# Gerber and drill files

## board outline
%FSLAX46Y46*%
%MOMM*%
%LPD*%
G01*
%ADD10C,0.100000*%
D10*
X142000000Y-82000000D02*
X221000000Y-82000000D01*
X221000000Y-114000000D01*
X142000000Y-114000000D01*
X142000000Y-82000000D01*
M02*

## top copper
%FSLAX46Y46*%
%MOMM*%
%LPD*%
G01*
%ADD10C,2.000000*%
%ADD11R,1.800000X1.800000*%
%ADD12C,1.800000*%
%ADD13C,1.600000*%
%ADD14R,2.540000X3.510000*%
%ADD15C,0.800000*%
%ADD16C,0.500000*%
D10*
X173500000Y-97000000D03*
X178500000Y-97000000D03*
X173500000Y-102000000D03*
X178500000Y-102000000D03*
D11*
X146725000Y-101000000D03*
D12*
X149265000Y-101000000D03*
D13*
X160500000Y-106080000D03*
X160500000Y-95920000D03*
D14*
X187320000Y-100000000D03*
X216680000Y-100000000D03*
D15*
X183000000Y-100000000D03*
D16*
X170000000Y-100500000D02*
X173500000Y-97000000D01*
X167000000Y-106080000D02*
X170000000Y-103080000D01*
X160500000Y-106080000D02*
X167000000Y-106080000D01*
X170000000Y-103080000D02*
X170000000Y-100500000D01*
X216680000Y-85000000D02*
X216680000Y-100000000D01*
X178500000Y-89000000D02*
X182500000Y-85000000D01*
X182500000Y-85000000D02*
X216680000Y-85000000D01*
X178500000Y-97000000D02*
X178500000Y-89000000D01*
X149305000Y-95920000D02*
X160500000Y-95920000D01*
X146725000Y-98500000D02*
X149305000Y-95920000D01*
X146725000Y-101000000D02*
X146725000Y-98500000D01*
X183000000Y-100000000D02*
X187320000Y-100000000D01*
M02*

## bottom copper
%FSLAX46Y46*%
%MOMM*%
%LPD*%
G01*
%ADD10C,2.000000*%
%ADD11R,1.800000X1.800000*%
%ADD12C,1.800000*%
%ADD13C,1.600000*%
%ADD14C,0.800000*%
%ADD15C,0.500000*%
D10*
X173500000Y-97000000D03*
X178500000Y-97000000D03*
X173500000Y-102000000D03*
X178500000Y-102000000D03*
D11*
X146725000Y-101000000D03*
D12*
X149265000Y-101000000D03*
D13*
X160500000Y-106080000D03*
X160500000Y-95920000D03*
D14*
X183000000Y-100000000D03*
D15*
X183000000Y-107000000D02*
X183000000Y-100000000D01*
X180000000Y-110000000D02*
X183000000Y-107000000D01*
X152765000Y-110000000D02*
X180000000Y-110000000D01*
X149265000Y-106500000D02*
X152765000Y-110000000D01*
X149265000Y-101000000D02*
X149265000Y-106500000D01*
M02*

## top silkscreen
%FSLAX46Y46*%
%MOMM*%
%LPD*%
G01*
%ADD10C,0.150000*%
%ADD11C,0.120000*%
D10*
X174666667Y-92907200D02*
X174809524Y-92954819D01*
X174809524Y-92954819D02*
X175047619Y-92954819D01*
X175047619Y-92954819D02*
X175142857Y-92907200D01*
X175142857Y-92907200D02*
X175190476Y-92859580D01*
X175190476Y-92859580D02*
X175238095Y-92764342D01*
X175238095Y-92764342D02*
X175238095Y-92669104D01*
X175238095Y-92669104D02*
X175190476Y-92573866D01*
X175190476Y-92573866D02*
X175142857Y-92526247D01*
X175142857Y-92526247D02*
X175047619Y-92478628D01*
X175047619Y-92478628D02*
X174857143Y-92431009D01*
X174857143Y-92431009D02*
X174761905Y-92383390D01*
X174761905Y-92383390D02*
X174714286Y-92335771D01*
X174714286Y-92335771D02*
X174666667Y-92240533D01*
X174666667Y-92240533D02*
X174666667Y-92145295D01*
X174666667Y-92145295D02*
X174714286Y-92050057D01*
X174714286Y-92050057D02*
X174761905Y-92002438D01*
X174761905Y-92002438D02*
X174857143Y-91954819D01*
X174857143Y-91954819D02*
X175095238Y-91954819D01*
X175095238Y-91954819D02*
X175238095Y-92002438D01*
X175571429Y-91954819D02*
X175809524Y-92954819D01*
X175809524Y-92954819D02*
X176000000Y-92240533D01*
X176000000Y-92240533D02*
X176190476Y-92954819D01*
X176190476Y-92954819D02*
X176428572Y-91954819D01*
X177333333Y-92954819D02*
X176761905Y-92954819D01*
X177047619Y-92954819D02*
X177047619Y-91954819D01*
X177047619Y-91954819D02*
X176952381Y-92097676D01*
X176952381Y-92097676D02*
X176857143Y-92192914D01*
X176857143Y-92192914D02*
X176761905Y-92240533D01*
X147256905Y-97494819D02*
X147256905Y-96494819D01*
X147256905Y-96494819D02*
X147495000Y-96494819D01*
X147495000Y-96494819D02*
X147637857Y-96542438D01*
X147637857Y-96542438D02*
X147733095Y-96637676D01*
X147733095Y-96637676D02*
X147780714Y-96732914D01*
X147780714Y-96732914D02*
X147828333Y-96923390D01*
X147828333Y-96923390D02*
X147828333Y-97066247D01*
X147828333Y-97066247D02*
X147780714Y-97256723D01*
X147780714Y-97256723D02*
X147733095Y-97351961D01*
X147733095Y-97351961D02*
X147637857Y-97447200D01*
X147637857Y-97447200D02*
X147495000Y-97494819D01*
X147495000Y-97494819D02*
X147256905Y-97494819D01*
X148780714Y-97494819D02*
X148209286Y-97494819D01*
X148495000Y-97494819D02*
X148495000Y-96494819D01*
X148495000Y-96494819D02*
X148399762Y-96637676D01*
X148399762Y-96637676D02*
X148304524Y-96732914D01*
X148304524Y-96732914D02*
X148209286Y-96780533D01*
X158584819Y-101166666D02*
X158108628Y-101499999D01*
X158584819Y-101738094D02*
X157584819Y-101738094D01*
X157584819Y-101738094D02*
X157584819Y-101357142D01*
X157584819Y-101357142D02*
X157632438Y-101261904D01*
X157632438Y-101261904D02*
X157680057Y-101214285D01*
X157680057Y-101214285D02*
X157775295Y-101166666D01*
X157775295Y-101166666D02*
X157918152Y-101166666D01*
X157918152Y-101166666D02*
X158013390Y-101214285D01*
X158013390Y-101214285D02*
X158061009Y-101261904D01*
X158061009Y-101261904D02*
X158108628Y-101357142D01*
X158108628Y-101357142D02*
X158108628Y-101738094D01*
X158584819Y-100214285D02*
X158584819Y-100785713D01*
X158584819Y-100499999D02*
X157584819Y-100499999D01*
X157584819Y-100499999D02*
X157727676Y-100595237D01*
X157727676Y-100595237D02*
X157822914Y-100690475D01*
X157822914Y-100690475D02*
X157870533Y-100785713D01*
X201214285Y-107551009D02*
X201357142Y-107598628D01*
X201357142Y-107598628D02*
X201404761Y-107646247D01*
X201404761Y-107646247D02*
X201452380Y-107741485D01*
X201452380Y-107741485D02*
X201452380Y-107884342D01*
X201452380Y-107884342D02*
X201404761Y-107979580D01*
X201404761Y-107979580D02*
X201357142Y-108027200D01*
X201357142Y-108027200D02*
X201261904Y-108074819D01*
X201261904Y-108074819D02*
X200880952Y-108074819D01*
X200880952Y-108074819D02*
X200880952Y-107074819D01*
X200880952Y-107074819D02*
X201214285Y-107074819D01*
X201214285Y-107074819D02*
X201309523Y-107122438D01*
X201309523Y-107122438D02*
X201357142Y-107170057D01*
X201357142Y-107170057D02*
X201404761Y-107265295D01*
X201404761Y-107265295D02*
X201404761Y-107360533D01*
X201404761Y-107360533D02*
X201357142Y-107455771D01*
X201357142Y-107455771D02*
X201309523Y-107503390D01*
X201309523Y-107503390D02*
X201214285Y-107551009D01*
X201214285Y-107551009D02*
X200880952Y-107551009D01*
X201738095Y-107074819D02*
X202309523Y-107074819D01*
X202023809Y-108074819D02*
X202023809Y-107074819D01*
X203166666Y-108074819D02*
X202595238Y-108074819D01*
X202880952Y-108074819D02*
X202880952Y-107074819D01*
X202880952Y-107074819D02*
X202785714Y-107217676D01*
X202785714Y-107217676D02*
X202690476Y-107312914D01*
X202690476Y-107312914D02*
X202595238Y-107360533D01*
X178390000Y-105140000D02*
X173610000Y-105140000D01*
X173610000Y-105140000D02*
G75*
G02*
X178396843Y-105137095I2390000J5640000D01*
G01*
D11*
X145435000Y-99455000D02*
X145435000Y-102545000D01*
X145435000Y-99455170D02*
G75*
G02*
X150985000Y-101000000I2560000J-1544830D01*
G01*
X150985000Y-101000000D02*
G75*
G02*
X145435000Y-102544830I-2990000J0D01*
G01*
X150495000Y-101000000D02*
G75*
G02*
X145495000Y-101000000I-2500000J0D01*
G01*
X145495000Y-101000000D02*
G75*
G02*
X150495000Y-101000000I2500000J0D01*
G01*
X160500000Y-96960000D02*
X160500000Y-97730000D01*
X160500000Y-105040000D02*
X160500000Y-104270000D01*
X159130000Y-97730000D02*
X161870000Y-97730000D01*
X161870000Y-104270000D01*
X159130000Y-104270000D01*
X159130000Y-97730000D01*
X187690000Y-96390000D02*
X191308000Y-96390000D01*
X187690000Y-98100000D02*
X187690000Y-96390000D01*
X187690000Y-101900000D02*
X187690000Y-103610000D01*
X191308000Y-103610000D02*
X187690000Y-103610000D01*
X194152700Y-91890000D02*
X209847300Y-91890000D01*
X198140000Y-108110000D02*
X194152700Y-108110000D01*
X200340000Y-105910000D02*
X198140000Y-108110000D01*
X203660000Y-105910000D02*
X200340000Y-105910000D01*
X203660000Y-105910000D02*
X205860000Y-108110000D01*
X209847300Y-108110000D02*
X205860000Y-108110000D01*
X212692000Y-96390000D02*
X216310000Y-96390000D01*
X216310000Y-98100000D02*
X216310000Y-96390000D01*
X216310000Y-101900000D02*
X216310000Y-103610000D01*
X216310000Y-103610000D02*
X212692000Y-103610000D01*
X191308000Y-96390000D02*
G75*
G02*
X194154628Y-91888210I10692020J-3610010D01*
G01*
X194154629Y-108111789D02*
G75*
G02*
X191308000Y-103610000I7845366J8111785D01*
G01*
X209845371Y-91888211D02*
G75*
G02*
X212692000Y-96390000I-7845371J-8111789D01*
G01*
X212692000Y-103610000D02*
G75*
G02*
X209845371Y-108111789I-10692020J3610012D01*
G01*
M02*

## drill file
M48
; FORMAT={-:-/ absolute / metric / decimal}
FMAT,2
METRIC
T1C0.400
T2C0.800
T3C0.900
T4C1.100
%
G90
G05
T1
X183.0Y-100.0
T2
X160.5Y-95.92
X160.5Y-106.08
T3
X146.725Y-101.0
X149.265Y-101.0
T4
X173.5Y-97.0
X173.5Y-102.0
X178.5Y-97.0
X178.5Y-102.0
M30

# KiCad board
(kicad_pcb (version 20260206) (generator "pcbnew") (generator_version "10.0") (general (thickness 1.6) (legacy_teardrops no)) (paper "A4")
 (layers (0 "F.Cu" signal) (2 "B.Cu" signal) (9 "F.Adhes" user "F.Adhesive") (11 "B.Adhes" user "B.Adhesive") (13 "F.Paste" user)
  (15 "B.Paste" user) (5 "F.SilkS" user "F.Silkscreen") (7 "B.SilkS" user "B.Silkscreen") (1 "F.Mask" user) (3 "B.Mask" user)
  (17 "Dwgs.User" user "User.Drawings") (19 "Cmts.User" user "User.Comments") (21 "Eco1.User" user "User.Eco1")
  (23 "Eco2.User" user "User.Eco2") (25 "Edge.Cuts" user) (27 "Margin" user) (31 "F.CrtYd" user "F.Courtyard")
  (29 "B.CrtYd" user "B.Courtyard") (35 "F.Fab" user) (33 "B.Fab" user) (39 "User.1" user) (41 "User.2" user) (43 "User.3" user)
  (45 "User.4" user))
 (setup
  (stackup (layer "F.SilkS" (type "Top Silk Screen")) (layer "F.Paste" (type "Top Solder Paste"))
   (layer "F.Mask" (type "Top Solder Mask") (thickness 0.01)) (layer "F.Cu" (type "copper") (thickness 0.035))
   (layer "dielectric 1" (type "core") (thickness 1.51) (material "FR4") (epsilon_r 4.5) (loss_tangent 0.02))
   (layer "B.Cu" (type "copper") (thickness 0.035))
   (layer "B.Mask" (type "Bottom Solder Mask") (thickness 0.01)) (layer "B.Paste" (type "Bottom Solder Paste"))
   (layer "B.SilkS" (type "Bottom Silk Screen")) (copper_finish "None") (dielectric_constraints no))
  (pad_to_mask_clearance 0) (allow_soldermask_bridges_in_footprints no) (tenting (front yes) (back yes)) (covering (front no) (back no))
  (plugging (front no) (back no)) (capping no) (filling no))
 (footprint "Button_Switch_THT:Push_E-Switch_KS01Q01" (layer "F.Cu") (at 173.5 97)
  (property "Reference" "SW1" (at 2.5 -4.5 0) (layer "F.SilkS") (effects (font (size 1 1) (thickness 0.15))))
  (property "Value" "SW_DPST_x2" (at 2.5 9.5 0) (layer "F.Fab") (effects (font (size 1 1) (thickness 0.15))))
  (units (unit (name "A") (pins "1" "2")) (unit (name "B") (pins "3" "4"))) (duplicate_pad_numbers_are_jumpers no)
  (fp_line (start 4.89 8.14) (end 0.11 8.14) (stroke (width 0.15) (type solid)) (layer "F.SilkS"))
  (fp_arc (start 0.11 8.14) (mid 2.496283 -3.625495) (end 4.896843 8.137095) (stroke (width 0.15) (type solid)) (layer "F.SilkS"))
  (pad "1" thru_hole circle (at 0 0) (size 2 2) (drill 1.1) (layers "*.Cu" "*.Mask") (remove_unused_layers no) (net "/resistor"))
  (pad "2" thru_hole circle (at 5 0) (size 2 2) (drill 1.1) (layers "*.Cu" "*.Mask") (remove_unused_layers no) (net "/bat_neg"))
  (pad "3" thru_hole circle (at 0 5) (size 2 2) (drill 1.1) (layers "*.Cu" "*.Mask") (remove_unused_layers no)
   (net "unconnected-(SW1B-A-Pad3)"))
  (pad "4" thru_hole circle (at 5 5) (size 2 2) (drill 1.1) (layers "*.Cu" "*.Mask") (remove_unused_layers no)
   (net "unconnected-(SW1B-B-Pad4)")))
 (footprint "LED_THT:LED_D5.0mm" (layer "F.Cu") (at 146.725 101)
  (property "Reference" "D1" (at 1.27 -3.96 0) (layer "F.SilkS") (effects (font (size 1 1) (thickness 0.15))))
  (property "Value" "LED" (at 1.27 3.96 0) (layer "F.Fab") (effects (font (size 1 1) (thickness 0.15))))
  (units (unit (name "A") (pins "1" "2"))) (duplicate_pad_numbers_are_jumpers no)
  (fp_line (start -1.29 -1.545) (end -1.29 1.545) (stroke (width 0.12) (type solid)) (layer "F.SilkS"))
  (fp_arc (start -1.29 -1.54483) (mid 2.071779 -2.880495) (end 4.26 0) (stroke (width 0.12) (type solid)) (layer "F.SilkS"))
  (fp_arc (start 4.26 0) (mid 2.071779 2.880495) (end -1.29 1.54483) (stroke (width 0.12) (type solid)) (layer "F.SilkS"))
  (fp_circle (center 1.27 0) (end 3.77 0) (stroke (width 0.12) (type solid)) (fill no) (layer "F.SilkS"))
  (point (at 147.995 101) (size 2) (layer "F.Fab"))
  (pad "1" thru_hole rect (at 0 0) (size 1.8 1.8) (drill 0.9) (layers "*.Cu" "*.Mask") (remove_unused_layers no) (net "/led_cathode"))
  (pad "2" thru_hole circle (at 2.54 0) (size 1.8 1.8) (drill 0.9) (layers "*.Cu" "*.Mask") (remove_unused_layers no) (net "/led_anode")))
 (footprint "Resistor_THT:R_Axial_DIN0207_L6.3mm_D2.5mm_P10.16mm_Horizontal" (layer "F.Cu") (at 160.5 106.08 90)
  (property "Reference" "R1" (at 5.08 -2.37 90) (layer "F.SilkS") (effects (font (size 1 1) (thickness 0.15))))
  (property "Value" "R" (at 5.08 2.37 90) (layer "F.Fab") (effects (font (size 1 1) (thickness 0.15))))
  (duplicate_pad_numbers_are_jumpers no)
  (fp_line (start 9.12 0) (end 8.35 0) (stroke (width 0.12) (type solid)) (layer "F.SilkS"))
  (fp_line (start 1.04 0) (end 1.81 0) (stroke (width 0.12) (type solid)) (layer "F.SilkS"))
  (fp_rect (start 1.81 -1.37) (end 8.35 1.37) (stroke (width 0.12) (type solid)) (fill no) (layer "F.SilkS"))
  (pad "1" thru_hole circle (at 0 0 90) (size 1.6 1.6) (drill 0.8) (layers "*.Cu" "*.Mask") (remove_unused_layers no) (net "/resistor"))
  (pad "2" thru_hole circle (at 10.16 0 90) (size 1.6 1.6) (drill 0.8) (layers "*.Cu" "*.Mask") (remove_unused_layers no)
   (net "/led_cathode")))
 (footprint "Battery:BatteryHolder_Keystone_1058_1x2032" (layer "F.Cu") (at 202 100)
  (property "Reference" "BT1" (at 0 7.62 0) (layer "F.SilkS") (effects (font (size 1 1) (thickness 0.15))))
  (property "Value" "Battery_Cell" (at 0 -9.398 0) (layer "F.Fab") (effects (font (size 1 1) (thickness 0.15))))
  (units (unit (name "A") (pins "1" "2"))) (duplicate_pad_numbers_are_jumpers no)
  (fp_line (start -14.31 -3.61) (end -10.692 -3.61) (stroke (width 0.12) (type solid)) (layer "F.SilkS"))
  (fp_line (start -14.31 -1.9) (end -14.31 -3.61) (stroke (width 0.12) (type solid)) (layer "F.SilkS"))
  (fp_line (start -14.31 1.9) (end -14.31 3.61) (stroke (width 0.12) (type solid)) (layer "F.SilkS"))
  (fp_line (start -10.692 3.61) (end -14.31 3.61) (stroke (width 0.12) (type solid)) (layer "F.SilkS"))
  (fp_line (start -7.8473 -8.11) (end 7.8473 -8.11) (stroke (width 0.12) (type solid)) (layer "F.SilkS"))
  (fp_line (start -3.86 8.11) (end -7.8473 8.11) (stroke (width 0.12) (type solid)) (layer "F.SilkS"))
  (fp_line (start -1.66 5.91) (end -3.86 8.11) (stroke (width 0.12) (type solid)) (layer "F.SilkS"))
  (fp_line (start 1.66 5.91) (end -1.66 5.91) (stroke (width 0.12) (type solid)) (layer "F.SilkS"))
  (fp_line (start 1.66 5.91) (end 3.86 8.11) (stroke (width 0.12) (type solid)) (layer "F.SilkS"))
  (fp_line (start 7.8473 8.11) (end 3.86 8.11) (stroke (width 0.12) (type solid)) (layer "F.SilkS"))
  (fp_line (start 10.692 -3.61) (end 14.31 -3.61) (stroke (width 0.12) (type solid)) (layer "F.SilkS"))
  (fp_line (start 14.31 -1.9) (end 14.31 -3.61) (stroke (width 0.12) (type solid)) (layer "F.SilkS"))
  (fp_line (start 14.31 1.9) (end 14.31 3.61) (stroke (width 0.12) (type solid)) (layer "F.SilkS"))
  (fp_line (start 14.31 3.61) (end 10.692 3.61) (stroke (width 0.12) (type solid)) (layer "F.SilkS"))
  (fp_arc (start -10.692 -3.61) (mid -9.538084 -6.031244) (end -7.845371 -8.111789) (stroke (width 0.12) (type solid)) (layer "F.SilkS"))
  (fp_arc (start -7.845371 8.111789) (mid -9.538085 6.031244) (end -10.692 3.61) (stroke (width 0.12) (type solid)) (layer "F.SilkS"))
  (fp_arc (start 7.845371 -8.111789) (mid 9.538085 -6.031244) (end 10.692 -3.61) (stroke (width 0.12) (type solid)) (layer "F.SilkS"))
  (fp_arc (start 10.692 3.61) (mid 9.538084 6.031244) (end 7.845371 8.111789) (stroke (width 0.12) (type solid)) (layer "F.SilkS"))
  (pad "1" smd rect (at -14.68 0) (size 2.54 3.51) (layers "F.Cu" "F.Mask" "F.Paste") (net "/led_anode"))
  (pad "2" smd rect (at 14.68 0) (size 2.54 3.51) (layers "F.Cu" "F.Mask" "F.Paste") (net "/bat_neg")))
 (gr_rect (start 142 82) (end 221 114) (stroke (width 0.1) (type default)) (fill no) (layer "Edge.Cuts"))
 (segment (start 170 100.5) (end 173.5 97) (width 0.5) (layer "F.Cu") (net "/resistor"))
 (segment (start 167 106.08) (end 170 103.08) (width 0.5) (layer "F.Cu") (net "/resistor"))
 (segment (start 160.5 106.08) (end 167 106.08) (width 0.5) (layer "F.Cu") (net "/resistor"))
 (segment (start 170 103.08) (end 170 100.5) (width 0.5) (layer "F.Cu") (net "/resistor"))
 (segment (start 216.68 85) (end 216.68 100) (width 0.5) (layer "F.Cu") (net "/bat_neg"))
 (segment (start 178.5 89) (end 182.5 85) (width 0.5) (layer "F.Cu") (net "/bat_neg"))
 (segment (start 182.5 85) (end 216.68 85) (width 0.5) (layer "F.Cu") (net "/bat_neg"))
 (segment (start 178.5 97) (end 178.5 89) (width 0.5) (layer "F.Cu") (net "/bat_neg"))
 (segment (start 149.305 95.92) (end 160.5 95.92) (width 0.5) (layer "F.Cu") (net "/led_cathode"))
 (segment (start 146.725 98.5) (end 149.305 95.92) (width 0.5) (layer "F.Cu") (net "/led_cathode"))
 (segment (start 146.725 101) (end 146.725 98.5) (width 0.5) (layer "F.Cu") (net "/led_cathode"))
 (segment (start 183 100) (end 187.32 100) (width 0.5) (layer "F.Cu") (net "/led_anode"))
 (via (at 183 100) (size 0.8) (drill 0.4) (layers "F.Cu" "B.Cu") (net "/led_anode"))
 (segment (start 183 107) (end 183 100) (width 0.5) (layer "B.Cu") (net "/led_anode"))
 (segment (start 180 110) (end 183 107) (width 0.5) (layer "B.Cu") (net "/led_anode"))
 (segment (start 152.765 110) (end 180 110) (width 0.5) (layer "B.Cu") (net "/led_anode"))
 (segment (start 149.265 106.5) (end 152.765 110) (width 0.5) (layer "B.Cu") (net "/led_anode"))
 (segment (start 149.265 101) (end 149.265 106.5) (width 0.5) (layer "B.Cu") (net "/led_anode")))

